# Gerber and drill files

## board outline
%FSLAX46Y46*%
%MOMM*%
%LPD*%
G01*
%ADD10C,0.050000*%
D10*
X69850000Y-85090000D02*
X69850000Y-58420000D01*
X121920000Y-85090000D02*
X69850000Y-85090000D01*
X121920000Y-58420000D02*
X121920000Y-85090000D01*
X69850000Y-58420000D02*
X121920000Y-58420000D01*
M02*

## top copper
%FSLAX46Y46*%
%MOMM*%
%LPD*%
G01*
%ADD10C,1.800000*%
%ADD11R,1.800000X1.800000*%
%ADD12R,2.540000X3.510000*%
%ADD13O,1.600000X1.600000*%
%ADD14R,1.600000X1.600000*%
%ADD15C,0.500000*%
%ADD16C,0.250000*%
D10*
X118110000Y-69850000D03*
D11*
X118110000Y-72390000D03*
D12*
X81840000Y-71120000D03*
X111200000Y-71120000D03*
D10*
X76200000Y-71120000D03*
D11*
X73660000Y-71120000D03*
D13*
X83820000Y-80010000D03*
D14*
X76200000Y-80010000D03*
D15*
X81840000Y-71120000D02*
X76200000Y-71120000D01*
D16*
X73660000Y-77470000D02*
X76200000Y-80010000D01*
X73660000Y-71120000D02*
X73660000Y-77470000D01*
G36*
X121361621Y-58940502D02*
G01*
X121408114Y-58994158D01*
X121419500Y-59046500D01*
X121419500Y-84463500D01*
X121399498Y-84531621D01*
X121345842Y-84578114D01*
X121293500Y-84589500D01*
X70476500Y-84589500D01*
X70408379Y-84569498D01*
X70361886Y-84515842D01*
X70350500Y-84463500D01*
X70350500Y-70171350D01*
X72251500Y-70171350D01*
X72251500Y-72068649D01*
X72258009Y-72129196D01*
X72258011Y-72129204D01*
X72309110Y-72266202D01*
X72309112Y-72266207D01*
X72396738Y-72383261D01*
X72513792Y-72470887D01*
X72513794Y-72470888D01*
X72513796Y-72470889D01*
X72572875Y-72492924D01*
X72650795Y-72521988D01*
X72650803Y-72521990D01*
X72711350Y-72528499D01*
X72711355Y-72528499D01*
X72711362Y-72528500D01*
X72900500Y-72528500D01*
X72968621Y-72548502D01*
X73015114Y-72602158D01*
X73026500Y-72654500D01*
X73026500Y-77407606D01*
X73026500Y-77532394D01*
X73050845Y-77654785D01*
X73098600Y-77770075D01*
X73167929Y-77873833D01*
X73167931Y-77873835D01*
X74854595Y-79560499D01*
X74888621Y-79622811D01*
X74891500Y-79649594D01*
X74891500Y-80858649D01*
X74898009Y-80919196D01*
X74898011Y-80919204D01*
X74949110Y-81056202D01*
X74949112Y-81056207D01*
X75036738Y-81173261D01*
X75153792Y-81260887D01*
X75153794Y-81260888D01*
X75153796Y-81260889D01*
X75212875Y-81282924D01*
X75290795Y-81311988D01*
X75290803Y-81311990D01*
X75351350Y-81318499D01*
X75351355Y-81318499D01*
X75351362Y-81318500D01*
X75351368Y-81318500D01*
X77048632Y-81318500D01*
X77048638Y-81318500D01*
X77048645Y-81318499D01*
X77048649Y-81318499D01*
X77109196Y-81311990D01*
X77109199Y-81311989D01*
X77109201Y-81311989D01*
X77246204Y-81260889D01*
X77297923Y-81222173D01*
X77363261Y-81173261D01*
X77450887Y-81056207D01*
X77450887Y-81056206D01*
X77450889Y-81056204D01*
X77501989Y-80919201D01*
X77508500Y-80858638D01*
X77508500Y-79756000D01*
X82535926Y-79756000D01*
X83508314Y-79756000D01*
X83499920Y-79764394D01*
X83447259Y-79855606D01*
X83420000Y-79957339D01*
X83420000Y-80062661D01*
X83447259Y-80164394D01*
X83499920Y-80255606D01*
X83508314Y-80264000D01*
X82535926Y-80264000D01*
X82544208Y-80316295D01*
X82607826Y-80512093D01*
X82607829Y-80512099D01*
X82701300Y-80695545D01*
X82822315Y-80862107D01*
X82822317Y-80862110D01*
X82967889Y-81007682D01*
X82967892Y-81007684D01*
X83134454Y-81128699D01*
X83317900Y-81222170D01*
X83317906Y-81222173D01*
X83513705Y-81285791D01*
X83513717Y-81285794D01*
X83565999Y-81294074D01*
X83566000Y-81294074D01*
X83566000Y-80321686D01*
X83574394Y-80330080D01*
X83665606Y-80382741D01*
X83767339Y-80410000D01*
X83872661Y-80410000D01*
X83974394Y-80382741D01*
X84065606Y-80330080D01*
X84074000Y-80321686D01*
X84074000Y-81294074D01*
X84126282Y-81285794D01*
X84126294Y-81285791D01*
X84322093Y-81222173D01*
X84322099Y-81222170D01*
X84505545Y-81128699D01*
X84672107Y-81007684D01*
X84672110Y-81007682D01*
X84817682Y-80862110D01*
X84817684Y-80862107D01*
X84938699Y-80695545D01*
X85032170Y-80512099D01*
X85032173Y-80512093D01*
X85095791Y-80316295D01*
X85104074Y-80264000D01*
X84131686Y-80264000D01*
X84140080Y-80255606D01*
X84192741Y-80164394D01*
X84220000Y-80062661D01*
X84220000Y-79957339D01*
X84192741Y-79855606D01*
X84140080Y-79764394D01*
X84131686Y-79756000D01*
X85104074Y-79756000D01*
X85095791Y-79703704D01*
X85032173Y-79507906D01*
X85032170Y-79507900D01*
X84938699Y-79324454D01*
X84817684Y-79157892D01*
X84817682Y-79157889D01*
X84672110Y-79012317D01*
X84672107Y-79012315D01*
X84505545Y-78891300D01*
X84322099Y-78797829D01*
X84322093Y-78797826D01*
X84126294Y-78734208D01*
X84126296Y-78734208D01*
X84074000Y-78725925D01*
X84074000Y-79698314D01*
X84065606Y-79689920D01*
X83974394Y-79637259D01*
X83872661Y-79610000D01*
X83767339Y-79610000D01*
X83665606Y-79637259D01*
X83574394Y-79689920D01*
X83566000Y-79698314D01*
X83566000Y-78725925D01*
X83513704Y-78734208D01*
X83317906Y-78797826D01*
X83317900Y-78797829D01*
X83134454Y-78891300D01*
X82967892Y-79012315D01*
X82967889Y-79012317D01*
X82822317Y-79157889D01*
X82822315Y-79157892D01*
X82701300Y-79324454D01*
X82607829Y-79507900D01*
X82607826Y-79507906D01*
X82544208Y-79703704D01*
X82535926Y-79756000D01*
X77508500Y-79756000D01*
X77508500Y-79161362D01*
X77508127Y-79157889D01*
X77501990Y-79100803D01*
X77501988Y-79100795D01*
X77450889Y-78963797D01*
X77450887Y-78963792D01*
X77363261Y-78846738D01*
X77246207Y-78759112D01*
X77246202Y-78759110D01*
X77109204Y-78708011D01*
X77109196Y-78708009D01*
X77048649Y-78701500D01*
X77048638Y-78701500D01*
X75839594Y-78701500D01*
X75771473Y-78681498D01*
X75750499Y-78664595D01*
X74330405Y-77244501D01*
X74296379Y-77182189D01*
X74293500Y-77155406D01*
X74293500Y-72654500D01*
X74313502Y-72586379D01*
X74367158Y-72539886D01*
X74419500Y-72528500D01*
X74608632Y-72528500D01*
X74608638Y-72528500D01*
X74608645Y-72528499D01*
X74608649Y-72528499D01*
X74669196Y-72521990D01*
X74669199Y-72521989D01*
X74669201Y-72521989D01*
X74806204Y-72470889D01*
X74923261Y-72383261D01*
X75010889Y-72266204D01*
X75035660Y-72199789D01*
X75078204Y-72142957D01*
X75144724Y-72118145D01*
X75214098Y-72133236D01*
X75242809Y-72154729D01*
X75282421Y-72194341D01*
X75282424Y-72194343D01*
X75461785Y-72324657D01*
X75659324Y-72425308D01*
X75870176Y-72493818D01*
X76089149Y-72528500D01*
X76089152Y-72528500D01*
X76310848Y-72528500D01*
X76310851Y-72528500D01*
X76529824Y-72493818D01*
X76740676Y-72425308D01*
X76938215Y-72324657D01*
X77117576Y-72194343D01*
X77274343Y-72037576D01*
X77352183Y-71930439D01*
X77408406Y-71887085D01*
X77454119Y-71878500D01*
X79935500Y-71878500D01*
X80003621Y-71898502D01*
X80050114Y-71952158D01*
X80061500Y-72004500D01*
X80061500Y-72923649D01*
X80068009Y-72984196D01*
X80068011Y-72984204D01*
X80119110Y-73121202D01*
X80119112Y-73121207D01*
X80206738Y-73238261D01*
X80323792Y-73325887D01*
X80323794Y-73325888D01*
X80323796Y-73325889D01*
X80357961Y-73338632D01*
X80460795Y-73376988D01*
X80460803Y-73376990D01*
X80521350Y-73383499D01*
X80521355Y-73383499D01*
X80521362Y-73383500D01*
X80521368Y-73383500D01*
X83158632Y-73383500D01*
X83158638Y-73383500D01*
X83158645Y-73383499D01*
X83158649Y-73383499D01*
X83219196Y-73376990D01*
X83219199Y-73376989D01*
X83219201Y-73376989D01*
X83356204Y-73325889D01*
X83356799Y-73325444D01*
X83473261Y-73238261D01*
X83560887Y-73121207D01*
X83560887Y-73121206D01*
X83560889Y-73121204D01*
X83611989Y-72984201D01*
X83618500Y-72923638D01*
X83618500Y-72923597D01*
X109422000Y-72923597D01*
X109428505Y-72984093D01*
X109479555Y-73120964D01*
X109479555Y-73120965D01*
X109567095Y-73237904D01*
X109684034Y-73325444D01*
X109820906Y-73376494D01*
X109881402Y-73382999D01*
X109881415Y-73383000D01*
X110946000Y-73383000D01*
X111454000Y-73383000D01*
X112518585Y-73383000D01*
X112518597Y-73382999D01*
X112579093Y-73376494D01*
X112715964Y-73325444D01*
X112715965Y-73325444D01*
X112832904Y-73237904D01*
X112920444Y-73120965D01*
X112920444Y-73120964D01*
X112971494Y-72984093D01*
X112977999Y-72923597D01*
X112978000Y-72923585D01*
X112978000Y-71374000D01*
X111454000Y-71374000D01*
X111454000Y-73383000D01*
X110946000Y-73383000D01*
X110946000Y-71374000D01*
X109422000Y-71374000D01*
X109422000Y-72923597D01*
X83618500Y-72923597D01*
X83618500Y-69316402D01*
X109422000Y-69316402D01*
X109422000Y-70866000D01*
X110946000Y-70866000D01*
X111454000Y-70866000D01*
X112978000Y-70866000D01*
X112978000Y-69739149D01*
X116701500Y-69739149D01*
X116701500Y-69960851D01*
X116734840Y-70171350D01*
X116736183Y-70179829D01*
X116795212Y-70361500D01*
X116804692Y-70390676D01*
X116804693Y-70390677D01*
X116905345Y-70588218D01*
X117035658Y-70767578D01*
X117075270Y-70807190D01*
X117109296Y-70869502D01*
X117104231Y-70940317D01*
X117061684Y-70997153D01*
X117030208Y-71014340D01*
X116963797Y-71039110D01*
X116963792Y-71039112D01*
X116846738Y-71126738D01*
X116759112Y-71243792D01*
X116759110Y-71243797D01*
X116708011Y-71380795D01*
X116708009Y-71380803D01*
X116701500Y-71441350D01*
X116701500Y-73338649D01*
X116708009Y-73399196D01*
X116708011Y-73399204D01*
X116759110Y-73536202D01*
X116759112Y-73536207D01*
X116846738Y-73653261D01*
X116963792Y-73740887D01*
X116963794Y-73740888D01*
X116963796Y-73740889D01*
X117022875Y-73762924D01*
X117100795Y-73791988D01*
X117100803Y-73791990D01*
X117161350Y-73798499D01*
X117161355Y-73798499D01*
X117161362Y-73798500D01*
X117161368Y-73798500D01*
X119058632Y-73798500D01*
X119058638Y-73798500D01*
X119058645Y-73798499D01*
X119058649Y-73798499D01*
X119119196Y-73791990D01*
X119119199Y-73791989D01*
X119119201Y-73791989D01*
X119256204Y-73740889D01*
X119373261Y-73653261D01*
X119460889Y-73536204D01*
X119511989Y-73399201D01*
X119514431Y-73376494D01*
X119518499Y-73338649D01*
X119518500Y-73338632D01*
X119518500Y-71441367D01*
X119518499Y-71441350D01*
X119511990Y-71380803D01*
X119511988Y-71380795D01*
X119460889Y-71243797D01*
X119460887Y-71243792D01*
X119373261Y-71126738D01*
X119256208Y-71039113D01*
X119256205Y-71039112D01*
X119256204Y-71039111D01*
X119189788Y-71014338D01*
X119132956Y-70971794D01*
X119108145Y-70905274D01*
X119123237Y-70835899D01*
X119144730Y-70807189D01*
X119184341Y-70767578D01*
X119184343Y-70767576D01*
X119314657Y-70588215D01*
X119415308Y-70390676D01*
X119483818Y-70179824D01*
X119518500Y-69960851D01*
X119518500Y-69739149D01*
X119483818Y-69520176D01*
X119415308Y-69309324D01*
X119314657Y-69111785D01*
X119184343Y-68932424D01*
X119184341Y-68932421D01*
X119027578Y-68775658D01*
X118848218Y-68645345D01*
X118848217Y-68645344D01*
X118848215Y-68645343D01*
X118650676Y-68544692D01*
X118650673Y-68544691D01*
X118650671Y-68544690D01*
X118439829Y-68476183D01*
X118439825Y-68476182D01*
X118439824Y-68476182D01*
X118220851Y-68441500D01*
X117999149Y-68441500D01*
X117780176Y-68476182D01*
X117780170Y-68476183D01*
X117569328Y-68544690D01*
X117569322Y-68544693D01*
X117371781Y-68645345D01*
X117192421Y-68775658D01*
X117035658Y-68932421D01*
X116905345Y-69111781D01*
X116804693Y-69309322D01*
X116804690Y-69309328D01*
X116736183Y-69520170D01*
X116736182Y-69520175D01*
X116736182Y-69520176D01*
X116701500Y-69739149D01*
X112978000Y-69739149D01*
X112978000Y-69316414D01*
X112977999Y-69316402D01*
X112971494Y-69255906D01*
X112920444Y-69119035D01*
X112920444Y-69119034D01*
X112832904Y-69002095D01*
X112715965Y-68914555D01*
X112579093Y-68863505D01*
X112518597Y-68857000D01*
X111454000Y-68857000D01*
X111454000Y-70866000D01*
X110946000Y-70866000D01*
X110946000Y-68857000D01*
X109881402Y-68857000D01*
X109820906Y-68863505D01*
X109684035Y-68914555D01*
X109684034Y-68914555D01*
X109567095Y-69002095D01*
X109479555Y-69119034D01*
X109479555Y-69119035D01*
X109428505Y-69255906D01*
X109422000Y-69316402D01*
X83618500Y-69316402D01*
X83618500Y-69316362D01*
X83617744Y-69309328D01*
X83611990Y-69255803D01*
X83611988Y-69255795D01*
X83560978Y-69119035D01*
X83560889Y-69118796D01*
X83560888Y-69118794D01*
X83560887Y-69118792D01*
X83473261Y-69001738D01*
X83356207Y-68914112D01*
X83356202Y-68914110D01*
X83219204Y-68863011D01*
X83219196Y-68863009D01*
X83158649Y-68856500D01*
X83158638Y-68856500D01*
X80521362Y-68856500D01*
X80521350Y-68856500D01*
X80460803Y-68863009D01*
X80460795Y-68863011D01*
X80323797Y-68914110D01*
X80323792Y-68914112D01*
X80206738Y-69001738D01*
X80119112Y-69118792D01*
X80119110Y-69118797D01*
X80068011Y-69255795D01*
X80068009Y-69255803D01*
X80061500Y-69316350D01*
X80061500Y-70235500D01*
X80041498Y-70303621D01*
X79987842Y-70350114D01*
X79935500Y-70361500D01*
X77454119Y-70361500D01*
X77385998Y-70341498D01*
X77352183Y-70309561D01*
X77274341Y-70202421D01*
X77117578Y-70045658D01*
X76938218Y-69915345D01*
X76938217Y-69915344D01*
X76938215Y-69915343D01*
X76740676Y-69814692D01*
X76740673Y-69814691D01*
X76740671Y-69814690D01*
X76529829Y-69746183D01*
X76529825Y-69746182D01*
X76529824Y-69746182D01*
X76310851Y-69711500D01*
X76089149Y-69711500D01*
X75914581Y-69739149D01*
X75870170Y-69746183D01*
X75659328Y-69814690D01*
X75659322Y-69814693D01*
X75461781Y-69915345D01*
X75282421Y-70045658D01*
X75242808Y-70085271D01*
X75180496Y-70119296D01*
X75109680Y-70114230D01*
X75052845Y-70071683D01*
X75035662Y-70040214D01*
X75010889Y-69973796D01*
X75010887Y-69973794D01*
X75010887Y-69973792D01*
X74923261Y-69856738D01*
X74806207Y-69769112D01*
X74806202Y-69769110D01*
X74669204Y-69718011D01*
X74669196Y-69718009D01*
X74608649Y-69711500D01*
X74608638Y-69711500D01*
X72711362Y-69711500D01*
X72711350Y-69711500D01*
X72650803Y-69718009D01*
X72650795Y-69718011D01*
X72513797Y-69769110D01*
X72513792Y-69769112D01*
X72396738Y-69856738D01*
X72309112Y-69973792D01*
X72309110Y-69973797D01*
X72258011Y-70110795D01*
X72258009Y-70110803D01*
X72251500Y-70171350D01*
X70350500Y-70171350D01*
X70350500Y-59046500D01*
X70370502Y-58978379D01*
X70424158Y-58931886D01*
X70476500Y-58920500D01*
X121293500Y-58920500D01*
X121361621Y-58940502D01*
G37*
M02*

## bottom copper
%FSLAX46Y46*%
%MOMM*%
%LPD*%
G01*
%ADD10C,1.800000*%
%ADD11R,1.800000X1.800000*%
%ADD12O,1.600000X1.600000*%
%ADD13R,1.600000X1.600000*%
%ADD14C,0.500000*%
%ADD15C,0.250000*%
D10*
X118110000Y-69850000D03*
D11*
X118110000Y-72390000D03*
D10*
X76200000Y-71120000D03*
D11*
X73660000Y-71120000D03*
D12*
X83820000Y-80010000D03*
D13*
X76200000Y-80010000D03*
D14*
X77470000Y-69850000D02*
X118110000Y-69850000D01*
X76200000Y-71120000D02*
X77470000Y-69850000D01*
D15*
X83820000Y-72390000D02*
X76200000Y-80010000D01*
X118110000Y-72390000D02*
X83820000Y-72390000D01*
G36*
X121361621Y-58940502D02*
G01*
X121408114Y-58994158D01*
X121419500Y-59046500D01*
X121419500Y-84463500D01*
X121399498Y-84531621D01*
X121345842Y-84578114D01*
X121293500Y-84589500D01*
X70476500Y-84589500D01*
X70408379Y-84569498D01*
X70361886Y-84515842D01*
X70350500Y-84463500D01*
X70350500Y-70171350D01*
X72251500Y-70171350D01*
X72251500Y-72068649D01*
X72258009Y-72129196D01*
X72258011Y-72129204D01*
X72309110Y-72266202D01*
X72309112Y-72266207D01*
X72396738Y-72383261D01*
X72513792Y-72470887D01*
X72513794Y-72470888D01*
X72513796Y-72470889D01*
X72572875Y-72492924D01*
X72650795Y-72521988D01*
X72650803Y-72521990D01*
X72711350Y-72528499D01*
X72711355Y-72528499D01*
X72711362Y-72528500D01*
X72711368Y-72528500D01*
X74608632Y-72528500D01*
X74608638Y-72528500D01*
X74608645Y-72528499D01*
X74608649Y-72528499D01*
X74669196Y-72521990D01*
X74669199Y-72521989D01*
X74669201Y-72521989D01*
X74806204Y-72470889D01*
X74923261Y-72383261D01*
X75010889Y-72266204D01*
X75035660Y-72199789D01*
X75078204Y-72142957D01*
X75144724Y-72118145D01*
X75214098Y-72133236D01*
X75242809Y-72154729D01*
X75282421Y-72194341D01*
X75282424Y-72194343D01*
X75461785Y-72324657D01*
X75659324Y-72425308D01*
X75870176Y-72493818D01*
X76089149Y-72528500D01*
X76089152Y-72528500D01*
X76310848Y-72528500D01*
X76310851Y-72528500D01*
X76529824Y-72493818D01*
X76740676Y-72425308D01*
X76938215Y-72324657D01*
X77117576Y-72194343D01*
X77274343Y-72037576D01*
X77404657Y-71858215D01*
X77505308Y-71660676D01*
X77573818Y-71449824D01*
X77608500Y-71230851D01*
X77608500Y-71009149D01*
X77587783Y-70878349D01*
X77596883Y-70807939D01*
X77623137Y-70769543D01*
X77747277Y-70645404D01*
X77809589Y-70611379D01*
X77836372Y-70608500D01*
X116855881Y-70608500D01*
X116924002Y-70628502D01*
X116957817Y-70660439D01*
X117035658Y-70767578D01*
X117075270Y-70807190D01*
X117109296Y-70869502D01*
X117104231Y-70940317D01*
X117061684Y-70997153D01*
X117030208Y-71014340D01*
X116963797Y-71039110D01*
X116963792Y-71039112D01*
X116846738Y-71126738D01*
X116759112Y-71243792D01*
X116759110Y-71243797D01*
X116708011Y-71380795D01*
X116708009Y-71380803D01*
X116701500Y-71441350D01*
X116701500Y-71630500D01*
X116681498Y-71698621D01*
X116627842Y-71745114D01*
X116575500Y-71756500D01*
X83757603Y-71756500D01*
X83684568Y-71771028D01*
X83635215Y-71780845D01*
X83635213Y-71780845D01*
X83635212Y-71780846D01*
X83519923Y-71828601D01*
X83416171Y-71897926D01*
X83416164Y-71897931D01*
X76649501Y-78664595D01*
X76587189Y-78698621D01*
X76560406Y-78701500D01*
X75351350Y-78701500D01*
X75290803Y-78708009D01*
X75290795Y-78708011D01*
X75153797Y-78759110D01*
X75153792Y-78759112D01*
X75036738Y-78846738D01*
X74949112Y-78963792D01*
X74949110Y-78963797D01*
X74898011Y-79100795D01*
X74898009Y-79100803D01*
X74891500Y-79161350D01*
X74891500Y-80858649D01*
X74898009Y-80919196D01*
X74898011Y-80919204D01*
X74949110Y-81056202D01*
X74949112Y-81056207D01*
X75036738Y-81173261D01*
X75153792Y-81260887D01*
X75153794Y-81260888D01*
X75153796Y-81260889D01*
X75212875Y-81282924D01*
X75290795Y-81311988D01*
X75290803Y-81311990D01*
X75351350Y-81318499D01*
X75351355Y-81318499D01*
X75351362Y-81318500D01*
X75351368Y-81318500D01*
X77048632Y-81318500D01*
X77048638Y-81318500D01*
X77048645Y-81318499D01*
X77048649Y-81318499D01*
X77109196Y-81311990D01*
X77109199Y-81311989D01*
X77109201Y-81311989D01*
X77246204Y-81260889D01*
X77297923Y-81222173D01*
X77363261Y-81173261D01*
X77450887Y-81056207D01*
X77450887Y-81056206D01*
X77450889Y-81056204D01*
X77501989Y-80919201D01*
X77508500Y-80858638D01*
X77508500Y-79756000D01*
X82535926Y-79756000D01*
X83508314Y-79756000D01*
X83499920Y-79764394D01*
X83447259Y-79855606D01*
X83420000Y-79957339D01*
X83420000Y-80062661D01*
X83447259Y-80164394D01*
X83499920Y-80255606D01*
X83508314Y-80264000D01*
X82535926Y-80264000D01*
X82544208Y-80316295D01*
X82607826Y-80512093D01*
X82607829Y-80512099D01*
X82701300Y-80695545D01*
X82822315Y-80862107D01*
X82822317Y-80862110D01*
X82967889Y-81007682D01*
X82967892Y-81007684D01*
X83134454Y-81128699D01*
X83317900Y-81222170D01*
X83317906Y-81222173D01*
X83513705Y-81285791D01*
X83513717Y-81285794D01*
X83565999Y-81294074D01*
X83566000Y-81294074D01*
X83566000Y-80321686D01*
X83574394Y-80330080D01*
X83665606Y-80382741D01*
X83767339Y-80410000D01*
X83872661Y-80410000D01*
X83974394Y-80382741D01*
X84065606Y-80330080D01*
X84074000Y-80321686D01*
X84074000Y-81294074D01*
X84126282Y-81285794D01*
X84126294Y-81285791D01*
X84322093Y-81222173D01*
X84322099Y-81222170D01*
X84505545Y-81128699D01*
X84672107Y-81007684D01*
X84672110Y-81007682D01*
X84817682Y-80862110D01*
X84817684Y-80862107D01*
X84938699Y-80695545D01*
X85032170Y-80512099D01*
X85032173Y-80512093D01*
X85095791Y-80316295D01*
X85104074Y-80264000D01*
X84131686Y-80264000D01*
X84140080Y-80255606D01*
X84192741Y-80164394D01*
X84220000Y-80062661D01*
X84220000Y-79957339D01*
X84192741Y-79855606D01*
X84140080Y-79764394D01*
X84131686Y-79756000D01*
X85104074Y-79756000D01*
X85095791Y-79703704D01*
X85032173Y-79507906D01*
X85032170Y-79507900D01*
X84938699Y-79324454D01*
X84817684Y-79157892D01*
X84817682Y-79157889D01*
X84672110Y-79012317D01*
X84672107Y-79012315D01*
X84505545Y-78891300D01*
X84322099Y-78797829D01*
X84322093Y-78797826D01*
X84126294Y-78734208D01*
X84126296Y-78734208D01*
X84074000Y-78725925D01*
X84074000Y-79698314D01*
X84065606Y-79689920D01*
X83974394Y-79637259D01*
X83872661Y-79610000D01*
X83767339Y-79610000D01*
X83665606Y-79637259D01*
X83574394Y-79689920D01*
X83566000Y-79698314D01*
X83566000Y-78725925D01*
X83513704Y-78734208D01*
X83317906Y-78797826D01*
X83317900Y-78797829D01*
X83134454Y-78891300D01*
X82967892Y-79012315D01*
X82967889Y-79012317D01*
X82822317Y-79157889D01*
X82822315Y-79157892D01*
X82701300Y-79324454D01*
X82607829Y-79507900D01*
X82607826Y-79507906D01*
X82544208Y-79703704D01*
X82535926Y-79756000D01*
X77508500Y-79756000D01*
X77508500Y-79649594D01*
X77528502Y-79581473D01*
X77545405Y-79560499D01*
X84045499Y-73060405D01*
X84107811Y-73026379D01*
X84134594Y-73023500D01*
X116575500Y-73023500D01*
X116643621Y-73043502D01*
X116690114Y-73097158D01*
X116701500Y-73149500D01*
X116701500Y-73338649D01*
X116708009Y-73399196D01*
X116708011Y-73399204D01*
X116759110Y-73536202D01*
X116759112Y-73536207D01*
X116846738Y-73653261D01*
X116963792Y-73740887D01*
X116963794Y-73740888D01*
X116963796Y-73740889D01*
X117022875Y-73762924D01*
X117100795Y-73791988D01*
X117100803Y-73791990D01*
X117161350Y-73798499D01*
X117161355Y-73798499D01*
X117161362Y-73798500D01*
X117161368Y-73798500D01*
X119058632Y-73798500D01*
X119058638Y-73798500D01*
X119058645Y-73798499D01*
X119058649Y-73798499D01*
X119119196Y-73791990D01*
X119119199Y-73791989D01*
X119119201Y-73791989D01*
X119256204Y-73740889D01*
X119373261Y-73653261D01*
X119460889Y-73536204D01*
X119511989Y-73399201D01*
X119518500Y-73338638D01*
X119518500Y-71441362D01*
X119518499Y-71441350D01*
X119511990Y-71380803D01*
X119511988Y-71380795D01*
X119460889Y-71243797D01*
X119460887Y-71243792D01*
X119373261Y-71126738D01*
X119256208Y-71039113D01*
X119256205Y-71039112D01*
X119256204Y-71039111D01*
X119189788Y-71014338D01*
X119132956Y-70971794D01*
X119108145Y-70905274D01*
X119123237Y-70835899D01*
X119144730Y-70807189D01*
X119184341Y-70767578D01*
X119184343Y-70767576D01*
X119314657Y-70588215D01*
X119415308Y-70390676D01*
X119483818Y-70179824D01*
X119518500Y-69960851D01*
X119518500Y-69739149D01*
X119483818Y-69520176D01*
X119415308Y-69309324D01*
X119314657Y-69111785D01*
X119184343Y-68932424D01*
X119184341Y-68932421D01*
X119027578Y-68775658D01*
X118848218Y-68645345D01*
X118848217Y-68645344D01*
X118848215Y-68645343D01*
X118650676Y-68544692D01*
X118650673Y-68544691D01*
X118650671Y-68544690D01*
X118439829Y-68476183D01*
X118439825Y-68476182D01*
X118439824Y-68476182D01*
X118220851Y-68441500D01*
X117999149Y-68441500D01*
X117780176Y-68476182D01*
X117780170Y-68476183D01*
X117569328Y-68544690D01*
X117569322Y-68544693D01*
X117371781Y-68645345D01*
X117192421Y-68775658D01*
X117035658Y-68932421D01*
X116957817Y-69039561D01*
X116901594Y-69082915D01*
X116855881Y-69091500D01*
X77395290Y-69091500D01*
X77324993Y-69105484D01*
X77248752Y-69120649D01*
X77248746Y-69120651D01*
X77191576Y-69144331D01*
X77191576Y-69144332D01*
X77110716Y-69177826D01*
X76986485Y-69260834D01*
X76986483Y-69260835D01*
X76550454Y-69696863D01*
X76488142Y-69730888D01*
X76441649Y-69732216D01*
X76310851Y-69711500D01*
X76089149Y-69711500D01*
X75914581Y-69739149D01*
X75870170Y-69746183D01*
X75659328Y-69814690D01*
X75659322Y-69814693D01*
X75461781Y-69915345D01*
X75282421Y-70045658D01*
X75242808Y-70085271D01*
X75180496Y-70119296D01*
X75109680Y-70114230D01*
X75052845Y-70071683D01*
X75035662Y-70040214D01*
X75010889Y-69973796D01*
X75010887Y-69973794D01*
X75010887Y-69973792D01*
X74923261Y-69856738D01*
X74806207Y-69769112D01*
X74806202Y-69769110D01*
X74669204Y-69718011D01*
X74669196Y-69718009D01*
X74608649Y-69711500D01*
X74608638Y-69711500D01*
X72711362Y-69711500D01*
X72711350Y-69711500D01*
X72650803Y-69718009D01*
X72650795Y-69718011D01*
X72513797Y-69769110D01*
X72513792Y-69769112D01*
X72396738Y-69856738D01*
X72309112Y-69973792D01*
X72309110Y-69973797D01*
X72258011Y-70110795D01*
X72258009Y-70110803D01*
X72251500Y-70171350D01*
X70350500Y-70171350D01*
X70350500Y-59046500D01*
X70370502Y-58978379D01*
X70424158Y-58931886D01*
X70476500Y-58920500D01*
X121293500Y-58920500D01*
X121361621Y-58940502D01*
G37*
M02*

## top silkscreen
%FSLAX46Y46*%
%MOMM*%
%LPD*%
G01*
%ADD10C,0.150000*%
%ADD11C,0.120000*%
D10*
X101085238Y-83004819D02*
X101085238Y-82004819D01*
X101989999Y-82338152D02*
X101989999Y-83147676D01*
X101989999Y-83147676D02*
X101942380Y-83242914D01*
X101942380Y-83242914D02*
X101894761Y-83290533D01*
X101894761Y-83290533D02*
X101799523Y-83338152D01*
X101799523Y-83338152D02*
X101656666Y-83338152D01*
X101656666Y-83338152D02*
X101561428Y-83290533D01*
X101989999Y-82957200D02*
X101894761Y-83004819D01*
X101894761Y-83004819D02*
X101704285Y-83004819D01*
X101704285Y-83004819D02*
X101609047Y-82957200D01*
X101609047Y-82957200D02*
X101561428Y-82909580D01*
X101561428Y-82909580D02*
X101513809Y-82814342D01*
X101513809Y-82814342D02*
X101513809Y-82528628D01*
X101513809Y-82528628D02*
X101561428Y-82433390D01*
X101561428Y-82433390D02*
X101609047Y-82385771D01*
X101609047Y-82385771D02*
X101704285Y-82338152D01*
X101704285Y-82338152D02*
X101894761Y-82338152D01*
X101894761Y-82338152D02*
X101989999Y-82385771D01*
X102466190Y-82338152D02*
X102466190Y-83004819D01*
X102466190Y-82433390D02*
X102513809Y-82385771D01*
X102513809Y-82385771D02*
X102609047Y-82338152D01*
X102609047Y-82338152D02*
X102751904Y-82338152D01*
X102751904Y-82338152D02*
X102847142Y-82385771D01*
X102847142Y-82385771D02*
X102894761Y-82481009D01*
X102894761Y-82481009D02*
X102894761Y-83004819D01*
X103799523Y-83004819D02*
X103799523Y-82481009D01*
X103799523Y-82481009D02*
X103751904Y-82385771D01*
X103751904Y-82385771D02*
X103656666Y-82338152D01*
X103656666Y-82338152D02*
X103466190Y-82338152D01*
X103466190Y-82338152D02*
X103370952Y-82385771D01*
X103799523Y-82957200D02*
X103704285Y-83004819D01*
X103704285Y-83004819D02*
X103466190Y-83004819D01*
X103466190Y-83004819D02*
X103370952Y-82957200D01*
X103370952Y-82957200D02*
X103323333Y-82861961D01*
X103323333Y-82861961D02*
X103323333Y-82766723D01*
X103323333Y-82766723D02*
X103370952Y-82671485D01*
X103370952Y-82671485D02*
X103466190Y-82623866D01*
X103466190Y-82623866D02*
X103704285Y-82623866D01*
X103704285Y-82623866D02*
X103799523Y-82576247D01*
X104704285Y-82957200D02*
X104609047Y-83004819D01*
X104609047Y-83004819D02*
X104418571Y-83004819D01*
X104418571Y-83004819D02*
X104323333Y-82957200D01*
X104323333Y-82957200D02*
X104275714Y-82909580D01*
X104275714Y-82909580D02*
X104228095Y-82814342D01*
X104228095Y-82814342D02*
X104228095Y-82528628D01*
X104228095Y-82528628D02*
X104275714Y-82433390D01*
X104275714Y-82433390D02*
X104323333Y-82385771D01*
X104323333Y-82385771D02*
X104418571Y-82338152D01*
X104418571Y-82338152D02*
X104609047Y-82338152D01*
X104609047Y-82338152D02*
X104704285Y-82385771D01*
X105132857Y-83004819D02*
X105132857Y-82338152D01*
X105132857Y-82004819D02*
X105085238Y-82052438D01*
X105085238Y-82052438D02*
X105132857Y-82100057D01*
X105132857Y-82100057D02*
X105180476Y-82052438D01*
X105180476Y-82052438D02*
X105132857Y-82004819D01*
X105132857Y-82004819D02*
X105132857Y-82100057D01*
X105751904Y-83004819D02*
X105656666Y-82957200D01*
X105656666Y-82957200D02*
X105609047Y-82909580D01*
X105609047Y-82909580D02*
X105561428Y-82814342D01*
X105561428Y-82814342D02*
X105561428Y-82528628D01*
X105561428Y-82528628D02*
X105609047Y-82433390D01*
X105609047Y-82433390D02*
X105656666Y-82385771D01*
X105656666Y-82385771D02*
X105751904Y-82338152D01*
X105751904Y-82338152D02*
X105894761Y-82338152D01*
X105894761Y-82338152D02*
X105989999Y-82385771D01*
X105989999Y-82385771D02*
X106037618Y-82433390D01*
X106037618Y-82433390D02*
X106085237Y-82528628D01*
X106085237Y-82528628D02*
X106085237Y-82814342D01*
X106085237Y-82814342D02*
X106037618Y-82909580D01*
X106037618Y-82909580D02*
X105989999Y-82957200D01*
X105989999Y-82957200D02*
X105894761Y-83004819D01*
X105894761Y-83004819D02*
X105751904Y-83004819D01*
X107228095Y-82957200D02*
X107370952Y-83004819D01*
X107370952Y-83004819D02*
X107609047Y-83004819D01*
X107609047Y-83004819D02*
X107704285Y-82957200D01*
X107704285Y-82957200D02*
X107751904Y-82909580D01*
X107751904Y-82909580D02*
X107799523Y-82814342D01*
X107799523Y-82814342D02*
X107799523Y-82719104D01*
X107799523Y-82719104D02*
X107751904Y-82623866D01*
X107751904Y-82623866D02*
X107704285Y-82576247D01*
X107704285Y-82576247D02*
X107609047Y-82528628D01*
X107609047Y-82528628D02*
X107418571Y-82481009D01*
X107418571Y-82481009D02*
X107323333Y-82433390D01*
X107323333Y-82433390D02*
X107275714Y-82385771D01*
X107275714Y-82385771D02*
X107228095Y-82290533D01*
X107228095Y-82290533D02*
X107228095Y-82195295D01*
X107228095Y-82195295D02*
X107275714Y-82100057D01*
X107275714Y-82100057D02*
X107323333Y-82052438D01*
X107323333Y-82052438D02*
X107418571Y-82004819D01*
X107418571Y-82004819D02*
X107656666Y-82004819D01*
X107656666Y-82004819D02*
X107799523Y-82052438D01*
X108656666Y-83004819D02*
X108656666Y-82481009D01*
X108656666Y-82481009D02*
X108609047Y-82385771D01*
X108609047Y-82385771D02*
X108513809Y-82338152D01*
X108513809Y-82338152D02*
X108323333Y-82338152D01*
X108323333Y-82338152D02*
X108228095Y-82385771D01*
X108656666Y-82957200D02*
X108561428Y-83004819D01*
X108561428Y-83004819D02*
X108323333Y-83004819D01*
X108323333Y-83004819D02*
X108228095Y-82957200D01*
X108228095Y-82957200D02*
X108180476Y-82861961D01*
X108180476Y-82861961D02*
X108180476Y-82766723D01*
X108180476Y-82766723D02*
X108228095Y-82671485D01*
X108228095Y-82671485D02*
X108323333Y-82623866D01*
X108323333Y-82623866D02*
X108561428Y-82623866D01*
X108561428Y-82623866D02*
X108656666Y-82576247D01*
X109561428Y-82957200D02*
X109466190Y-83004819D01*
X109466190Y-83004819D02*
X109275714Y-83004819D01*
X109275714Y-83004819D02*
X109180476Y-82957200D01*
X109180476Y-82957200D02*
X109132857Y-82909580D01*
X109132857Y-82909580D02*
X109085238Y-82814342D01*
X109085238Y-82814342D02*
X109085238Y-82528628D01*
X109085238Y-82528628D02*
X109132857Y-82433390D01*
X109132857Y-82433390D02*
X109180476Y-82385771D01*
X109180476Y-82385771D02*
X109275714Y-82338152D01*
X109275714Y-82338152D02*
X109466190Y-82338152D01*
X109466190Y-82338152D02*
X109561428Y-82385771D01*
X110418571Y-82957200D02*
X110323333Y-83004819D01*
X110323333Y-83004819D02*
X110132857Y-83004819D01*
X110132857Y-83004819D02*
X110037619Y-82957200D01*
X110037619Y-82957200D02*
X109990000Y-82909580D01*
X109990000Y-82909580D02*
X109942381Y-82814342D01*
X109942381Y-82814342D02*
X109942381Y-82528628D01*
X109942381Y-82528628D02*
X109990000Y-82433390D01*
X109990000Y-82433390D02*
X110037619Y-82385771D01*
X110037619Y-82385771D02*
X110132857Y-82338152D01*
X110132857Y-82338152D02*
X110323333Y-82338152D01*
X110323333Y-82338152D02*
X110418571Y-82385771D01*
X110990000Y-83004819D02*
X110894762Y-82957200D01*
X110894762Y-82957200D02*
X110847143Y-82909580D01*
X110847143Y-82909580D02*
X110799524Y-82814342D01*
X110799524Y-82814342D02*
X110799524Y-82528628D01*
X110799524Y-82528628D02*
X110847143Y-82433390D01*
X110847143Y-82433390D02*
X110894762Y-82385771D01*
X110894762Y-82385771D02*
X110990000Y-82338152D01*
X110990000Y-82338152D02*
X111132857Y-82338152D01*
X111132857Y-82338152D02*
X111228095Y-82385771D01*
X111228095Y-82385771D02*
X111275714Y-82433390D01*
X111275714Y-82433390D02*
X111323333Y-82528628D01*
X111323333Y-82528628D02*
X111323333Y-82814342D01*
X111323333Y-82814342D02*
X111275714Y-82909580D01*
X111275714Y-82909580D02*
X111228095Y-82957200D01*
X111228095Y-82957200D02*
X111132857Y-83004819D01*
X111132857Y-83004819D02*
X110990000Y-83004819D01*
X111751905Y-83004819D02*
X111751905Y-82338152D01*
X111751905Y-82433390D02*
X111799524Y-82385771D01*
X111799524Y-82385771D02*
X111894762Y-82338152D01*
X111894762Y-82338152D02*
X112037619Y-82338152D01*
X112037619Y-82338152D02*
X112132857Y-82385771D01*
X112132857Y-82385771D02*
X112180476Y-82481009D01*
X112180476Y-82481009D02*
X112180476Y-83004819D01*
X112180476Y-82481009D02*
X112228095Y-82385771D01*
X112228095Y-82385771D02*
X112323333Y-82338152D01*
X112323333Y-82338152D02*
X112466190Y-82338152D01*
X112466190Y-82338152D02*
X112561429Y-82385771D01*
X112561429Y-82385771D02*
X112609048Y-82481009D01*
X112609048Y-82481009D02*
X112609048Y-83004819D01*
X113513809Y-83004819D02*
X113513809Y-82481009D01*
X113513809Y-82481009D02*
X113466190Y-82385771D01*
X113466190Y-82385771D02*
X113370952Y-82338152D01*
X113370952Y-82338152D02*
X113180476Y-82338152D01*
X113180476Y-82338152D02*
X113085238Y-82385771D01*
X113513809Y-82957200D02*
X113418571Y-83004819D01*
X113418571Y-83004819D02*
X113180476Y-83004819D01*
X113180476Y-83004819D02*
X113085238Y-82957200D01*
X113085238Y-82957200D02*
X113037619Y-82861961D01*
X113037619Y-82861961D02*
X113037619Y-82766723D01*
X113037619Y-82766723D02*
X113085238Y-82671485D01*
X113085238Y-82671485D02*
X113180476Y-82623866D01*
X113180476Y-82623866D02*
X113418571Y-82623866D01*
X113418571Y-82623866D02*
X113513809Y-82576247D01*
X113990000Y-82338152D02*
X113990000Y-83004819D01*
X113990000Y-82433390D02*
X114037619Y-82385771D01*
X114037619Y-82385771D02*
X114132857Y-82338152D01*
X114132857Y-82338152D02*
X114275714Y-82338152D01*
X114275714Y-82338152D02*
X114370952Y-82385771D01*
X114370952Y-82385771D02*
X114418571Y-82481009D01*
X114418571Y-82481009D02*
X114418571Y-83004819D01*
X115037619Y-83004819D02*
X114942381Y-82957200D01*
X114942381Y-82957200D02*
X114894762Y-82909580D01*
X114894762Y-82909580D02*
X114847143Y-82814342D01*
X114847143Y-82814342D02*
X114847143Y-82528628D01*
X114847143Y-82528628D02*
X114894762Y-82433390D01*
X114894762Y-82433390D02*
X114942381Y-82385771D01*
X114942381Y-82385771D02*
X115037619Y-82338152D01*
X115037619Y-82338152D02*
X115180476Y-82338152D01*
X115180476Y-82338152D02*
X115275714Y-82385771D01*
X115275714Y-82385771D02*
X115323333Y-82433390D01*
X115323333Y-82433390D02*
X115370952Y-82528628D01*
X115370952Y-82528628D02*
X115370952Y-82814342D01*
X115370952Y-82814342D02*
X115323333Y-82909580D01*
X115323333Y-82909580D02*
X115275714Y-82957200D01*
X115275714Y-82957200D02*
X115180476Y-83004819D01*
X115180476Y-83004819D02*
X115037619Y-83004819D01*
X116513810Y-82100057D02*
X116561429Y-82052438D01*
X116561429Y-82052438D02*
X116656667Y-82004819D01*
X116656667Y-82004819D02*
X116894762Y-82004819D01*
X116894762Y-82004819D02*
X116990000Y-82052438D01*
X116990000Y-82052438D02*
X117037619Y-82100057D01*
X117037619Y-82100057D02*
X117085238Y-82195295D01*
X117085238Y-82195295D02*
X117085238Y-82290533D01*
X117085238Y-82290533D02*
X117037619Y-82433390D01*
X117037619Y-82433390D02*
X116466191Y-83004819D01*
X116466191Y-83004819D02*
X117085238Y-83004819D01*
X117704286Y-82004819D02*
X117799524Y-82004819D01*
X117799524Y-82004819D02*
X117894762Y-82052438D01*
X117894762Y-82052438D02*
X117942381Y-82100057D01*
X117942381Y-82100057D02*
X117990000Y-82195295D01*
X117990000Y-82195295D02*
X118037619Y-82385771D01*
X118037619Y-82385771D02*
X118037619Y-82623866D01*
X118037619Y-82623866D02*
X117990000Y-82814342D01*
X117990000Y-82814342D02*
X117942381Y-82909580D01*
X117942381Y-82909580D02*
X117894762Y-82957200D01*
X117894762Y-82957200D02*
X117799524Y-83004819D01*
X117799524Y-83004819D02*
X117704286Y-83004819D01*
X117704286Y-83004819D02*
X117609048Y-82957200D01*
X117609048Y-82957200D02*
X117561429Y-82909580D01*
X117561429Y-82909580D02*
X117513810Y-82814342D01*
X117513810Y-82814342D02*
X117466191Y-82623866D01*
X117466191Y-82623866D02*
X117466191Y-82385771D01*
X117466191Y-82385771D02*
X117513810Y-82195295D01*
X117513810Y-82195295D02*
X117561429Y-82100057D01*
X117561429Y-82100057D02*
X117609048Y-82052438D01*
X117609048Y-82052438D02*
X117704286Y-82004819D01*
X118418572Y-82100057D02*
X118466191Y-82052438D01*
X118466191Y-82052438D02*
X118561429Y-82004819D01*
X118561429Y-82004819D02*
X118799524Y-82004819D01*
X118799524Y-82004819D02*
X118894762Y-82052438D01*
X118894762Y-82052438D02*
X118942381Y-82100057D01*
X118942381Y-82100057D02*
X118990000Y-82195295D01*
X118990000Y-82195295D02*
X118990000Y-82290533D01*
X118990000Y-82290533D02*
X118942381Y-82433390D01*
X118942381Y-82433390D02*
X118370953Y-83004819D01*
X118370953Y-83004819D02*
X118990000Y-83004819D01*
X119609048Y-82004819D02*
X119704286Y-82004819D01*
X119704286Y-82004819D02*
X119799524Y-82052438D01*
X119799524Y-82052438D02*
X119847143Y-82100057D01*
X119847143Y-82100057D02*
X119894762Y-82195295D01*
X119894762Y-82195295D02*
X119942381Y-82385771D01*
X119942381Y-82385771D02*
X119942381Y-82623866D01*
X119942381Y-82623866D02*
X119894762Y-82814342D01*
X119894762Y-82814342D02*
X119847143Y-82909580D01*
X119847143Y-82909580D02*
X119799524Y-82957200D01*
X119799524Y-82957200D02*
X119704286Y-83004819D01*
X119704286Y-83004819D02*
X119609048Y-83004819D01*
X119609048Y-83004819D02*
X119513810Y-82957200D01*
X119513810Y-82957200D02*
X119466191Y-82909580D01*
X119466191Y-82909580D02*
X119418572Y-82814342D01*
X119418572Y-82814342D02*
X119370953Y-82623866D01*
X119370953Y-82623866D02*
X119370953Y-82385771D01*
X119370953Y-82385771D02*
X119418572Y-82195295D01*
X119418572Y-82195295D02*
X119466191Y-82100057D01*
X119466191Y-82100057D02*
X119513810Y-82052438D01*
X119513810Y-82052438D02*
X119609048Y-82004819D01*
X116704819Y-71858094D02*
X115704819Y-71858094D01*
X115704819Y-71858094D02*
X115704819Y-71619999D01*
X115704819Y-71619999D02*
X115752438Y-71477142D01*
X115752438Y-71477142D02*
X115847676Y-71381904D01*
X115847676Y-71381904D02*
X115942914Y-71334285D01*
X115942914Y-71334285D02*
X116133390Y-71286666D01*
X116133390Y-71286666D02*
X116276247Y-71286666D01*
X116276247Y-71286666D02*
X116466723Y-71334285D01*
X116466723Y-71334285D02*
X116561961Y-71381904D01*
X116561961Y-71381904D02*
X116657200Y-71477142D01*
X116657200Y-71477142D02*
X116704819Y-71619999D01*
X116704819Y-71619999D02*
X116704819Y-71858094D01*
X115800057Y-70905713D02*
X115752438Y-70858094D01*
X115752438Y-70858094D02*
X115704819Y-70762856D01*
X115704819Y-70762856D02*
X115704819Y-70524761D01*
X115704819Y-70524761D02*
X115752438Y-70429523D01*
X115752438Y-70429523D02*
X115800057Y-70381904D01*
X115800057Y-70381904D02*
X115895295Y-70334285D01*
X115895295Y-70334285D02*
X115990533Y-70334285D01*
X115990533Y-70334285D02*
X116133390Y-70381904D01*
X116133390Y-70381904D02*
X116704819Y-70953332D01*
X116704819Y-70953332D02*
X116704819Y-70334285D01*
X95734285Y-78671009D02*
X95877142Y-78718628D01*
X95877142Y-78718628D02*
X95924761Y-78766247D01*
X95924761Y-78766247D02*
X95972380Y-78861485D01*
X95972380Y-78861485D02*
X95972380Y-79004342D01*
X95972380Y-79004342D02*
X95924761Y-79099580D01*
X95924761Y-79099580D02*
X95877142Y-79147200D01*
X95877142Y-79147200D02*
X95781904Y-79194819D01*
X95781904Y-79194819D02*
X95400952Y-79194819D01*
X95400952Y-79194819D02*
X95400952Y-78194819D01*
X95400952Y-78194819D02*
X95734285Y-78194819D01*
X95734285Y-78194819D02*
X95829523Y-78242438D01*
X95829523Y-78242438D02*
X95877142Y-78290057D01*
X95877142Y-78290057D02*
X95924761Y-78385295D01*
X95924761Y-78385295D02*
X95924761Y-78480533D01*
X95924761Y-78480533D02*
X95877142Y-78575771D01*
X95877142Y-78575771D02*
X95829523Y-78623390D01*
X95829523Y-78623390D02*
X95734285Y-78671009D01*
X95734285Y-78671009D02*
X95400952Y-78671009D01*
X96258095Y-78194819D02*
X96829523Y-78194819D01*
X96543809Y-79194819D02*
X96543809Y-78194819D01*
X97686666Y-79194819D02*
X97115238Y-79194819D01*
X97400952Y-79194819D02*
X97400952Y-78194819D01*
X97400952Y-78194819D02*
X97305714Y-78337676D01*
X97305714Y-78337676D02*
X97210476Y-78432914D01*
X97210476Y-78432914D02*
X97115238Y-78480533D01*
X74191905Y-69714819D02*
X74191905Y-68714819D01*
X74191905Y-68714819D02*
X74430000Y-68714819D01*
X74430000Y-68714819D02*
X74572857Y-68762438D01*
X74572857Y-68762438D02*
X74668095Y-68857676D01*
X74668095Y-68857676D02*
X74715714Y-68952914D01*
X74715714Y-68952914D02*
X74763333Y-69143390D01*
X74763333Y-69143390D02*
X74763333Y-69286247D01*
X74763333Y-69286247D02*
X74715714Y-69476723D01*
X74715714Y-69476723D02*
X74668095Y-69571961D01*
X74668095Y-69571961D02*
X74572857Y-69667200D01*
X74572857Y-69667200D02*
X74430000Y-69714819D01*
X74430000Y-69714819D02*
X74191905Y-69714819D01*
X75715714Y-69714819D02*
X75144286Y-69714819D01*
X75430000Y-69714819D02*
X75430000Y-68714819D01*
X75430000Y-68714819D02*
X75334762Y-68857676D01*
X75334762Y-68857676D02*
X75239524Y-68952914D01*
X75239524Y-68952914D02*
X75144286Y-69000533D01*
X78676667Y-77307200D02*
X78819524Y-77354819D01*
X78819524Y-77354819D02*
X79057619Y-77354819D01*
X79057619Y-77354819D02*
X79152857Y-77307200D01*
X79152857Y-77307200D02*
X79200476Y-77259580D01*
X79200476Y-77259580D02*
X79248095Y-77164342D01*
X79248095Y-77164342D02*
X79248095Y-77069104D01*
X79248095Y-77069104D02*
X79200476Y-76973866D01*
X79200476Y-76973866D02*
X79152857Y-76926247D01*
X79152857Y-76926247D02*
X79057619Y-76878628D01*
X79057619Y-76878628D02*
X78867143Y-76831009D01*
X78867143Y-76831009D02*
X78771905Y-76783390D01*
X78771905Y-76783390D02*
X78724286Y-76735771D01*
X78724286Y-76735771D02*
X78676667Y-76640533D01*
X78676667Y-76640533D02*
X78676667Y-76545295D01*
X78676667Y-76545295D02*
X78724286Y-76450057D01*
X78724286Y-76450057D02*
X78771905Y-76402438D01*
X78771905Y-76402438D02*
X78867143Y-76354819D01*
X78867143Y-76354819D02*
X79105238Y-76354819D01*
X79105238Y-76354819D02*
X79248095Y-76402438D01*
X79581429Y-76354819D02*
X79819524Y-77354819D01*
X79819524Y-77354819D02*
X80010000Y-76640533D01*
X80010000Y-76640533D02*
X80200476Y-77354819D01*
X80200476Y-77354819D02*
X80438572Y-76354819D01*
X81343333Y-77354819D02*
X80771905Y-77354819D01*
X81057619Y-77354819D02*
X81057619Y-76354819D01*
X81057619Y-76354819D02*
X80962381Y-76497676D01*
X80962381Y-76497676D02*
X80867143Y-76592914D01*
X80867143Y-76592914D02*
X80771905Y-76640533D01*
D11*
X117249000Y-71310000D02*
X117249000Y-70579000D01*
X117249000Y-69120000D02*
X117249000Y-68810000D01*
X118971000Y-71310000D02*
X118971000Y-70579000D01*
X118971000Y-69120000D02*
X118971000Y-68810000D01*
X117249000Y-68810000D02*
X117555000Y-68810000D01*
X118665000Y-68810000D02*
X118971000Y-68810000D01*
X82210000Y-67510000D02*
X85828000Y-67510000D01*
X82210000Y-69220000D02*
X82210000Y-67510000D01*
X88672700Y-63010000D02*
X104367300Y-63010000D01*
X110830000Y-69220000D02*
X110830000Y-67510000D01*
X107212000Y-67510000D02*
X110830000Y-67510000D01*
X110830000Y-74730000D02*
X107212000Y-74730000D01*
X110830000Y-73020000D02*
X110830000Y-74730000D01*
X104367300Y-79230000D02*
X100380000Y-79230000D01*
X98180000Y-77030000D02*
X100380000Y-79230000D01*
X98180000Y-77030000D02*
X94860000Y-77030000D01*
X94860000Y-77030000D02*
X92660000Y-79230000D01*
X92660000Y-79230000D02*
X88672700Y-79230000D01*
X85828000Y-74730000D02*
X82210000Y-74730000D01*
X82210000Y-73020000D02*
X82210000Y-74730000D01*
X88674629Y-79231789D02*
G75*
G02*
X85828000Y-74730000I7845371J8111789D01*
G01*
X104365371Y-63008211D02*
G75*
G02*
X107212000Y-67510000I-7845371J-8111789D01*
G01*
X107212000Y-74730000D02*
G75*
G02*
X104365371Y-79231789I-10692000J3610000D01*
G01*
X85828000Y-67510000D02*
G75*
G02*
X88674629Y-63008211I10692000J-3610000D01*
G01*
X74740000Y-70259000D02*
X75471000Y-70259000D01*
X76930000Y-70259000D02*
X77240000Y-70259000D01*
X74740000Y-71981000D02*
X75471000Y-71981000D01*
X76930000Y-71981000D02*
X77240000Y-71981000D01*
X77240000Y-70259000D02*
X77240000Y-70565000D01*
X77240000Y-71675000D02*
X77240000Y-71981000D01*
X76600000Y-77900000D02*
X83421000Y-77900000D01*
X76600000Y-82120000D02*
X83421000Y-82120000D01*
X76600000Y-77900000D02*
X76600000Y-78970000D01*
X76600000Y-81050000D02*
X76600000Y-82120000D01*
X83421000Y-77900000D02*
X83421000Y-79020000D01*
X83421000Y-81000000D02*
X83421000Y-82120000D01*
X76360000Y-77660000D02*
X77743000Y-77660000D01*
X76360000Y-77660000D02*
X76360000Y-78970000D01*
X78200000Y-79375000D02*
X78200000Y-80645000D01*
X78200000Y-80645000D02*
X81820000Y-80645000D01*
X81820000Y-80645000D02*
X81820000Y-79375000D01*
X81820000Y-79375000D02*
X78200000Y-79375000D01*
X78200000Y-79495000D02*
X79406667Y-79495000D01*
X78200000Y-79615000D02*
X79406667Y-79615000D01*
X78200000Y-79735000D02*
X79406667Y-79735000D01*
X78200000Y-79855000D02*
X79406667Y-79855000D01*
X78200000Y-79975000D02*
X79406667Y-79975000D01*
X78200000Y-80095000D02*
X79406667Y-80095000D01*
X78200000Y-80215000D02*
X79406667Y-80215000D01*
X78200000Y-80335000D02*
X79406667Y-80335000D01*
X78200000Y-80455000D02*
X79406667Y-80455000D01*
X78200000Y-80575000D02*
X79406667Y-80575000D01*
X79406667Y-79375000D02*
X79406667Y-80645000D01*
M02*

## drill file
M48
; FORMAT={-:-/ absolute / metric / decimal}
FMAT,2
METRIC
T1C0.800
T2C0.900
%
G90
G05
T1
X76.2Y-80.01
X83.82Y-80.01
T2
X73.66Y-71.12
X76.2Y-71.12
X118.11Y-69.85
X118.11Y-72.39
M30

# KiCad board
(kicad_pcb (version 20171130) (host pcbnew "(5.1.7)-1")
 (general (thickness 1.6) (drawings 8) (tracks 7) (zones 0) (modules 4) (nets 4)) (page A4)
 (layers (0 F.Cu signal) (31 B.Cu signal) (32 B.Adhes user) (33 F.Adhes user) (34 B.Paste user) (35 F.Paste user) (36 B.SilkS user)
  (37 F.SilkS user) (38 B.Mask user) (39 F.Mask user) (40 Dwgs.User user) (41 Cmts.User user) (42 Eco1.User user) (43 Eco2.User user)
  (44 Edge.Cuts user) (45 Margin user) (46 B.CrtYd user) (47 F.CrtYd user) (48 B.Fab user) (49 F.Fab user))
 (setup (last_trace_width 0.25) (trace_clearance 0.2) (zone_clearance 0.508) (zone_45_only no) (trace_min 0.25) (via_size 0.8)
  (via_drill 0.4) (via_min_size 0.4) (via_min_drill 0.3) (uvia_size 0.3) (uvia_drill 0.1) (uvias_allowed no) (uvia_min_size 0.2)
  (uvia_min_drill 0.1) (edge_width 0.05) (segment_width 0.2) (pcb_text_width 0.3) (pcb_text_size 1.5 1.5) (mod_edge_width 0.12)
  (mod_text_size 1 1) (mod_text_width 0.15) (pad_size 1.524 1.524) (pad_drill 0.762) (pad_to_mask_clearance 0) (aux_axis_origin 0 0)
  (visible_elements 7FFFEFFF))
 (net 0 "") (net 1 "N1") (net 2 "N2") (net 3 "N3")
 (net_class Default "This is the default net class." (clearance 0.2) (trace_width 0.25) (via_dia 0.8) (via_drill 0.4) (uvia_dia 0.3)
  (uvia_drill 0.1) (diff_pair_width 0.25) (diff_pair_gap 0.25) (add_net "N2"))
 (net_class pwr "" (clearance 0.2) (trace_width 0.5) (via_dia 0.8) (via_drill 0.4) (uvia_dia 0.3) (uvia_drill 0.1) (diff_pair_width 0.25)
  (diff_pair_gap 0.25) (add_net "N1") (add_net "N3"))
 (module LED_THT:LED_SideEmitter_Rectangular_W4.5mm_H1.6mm (layer F.Cu) (at 118.11 72.39 90)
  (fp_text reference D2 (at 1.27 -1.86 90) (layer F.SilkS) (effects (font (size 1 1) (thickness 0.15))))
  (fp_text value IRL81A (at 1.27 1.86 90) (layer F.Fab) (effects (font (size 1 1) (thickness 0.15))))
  (fp_line (start 1.08 -0.861) (end 1.811 -0.861) (layer F.SilkS) (width 0.12))
  (fp_line (start 3.27 -0.861) (end 3.58 -0.861) (layer F.SilkS) (width 0.12))
  (fp_line (start 1.08 0.861) (end 1.811 0.861) (layer F.SilkS) (width 0.12))
  (fp_line (start 3.27 0.861) (end 3.58 0.861) (layer F.SilkS) (width 0.12))
  (fp_line (start 3.58 -0.861) (end 3.58 -0.555) (layer F.SilkS) (width 0.12))
  (fp_line (start 3.58 0.555) (end 3.58 0.861) (layer F.SilkS) (width 0.12))
  (pad 2 thru_hole circle (at 2.54 0 90) (size 1.8 1.8) (drill 0.9) (layers *.Cu *.Mask) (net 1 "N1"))
  (pad 1 thru_hole rect (at 0 0 90) (size 1.8 1.8) (drill 0.9) (layers *.Cu *.Mask) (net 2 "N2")))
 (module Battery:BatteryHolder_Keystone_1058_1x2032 (layer F.Cu) (at 96.52 71.12)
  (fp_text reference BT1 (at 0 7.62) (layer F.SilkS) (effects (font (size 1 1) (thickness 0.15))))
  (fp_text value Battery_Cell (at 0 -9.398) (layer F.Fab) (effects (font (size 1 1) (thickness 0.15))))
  (fp_line (start -14.31 -3.61) (end -10.692 -3.61) (layer F.SilkS) (width 0.12))
  (fp_line (start -14.31 -1.9) (end -14.31 -3.61) (layer F.SilkS) (width 0.12))
  (fp_line (start -7.8473 -8.11) (end 7.8473 -8.11) (layer F.SilkS) (width 0.12))
  (fp_line (start 14.31 -1.9) (end 14.31 -3.61) (layer F.SilkS) (width 0.12))
  (fp_line (start 10.692 -3.61) (end 14.31 -3.61) (layer F.SilkS) (width 0.12))
  (fp_line (start 14.31 3.61) (end 10.692 3.61) (layer F.SilkS) (width 0.12))
  (fp_line (start 14.31 1.9) (end 14.31 3.61) (layer F.SilkS) (width 0.12))
  (fp_line (start 7.8473 8.11) (end 3.86 8.11) (layer F.SilkS) (width 0.12))
  (fp_line (start 1.66 5.91) (end 3.86 8.11) (layer F.SilkS) (width 0.12))
  (fp_line (start 1.66 5.91) (end -1.66 5.91) (layer F.SilkS) (width 0.12))
  (fp_line (start -1.66 5.91) (end -3.86 8.11) (layer F.SilkS) (width 0.12))
  (fp_line (start -3.86 8.11) (end -7.8473 8.11) (layer F.SilkS) (width 0.12))
  (fp_line (start -10.692 3.61) (end -14.31 3.61) (layer F.SilkS) (width 0.12))
  (fp_line (start -14.31 1.9) (end -14.31 3.61) (layer F.SilkS) (width 0.12))
  (fp_arc (start 0 0) (end -10.692 3.61) (angle -27.3) (layer F.SilkS) (width 0.12))
  (fp_arc (start 0 0) (end 10.692 -3.61) (angle -27.3) (layer F.SilkS) (width 0.12))
  (fp_arc (start 0 0) (end 10.692 3.61) (angle 27.3) (layer F.SilkS) (width 0.12))
  (fp_arc (start 0 0) (end -10.692 -3.61) (angle 27.3) (layer F.SilkS) (width 0.12))
  (pad 1 smd rect (at -14.68 0) (size 2.54 3.51) (layers F.Cu F.Paste F.Mask) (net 1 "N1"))
  (pad 2 smd rect (at 14.68 0) (size 2.54 3.51) (layers F.Cu F.Paste F.Mask) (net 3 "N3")))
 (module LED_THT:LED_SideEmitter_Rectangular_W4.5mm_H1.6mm (layer F.Cu) (at 73.66 71.12)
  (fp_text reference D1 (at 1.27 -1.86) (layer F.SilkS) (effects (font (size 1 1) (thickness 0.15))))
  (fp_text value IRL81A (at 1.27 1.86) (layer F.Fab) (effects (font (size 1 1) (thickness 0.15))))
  (fp_line (start 1.08 -0.861) (end 1.811 -0.861) (layer F.SilkS) (width 0.12))
  (fp_line (start 3.27 -0.861) (end 3.58 -0.861) (layer F.SilkS) (width 0.12))
  (fp_line (start 1.08 0.861) (end 1.811 0.861) (layer F.SilkS) (width 0.12))
  (fp_line (start 3.27 0.861) (end 3.58 0.861) (layer F.SilkS) (width 0.12))
  (fp_line (start 3.58 -0.861) (end 3.58 -0.555) (layer F.SilkS) (width 0.12))
  (fp_line (start 3.58 0.555) (end 3.58 0.861) (layer F.SilkS) (width 0.12))
  (pad 2 thru_hole circle (at 2.54 0) (size 1.8 1.8) (drill 0.9) (layers *.Cu *.Mask) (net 1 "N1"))
  (pad 1 thru_hole rect (at 0 0) (size 1.8 1.8) (drill 0.9) (layers *.Cu *.Mask) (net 2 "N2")))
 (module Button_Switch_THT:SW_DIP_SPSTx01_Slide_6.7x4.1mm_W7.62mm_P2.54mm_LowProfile (layer F.Cu) (at 76.2 80.01)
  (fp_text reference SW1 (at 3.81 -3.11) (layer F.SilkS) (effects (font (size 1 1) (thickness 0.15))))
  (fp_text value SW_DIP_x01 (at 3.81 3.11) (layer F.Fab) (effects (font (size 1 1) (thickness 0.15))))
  (fp_line (start 0.4 -2.11) (end 7.221 -2.11) (layer F.SilkS) (width 0.12))
  (fp_line (start 0.4 2.11) (end 7.221 2.11) (layer F.SilkS) (width 0.12))
  (fp_line (start 0.4 -2.11) (end 0.4 -1.04) (layer F.SilkS) (width 0.12))
  (fp_line (start 0.4 1.04) (end 0.4 2.11) (layer F.SilkS) (width 0.12))
  (fp_line (start 7.221 -2.11) (end 7.221 -0.99) (layer F.SilkS) (width 0.12))
  (fp_line (start 7.221 0.99) (end 7.221 2.11) (layer F.SilkS) (width 0.12))
  (fp_line (start 0.16 -2.35) (end 1.543 -2.35) (layer F.SilkS) (width 0.12))
  (fp_line (start 0.16 -2.35) (end 0.16 -1.04) (layer F.SilkS) (width 0.12))
  (fp_line (start 2 -0.635) (end 2 0.635) (layer F.SilkS) (width 0.12))
  (fp_line (start 2 0.635) (end 5.62 0.635) (layer F.SilkS) (width 0.12))
  (fp_line (start 5.62 0.635) (end 5.62 -0.635) (layer F.SilkS) (width 0.12))
  (fp_line (start 5.62 -0.635) (end 2 -0.635) (layer F.SilkS) (width 0.12))
  (fp_line (start 2 -0.515) (end 3.206667 -0.515) (layer F.SilkS) (width 0.12))
  (fp_line (start 2 -0.395) (end 3.206667 -0.395) (layer F.SilkS) (width 0.12))
  (fp_line (start 2 -0.275) (end 3.206667 -0.275) (layer F.SilkS) (width 0.12))
  (fp_line (start 2 -0.155) (end 3.206667 -0.155) (layer F.SilkS) (width 0.12))
  (fp_line (start 2 -0.035) (end 3.206667 -0.035) (layer F.SilkS) (width 0.12))
  (fp_line (start 2 0.085) (end 3.206667 0.085) (layer F.SilkS) (width 0.12))
  (fp_line (start 2 0.205) (end 3.206667 0.205) (layer F.SilkS) (width 0.12))
  (fp_line (start 2 0.325) (end 3.206667 0.325) (layer F.SilkS) (width 0.12))
  (fp_line (start 2 0.445) (end 3.206667 0.445) (layer F.SilkS) (width 0.12))
  (fp_line (start 2 0.565) (end 3.206667 0.565) (layer F.SilkS) (width 0.12))
  (fp_line (start 3.206667 -0.635) (end 3.206667 0.635) (layer F.SilkS) (width 0.12))
  (pad 2 thru_hole oval (at 7.62 0) (size 1.6 1.6) (drill 0.8) (layers *.Cu *.Mask) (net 3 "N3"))
  (pad 1 thru_hole rect (at 0 0) (size 1.6 1.6) (drill 0.8) (layers *.Cu *.Mask) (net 2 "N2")))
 (gr_line (start 69.85 85.09) (end 69.85 58.42) (layer Edge.Cuts) (width 0.05))
 (gr_line (start 121.92 85.09) (end 69.85 85.09) (layer Edge.Cuts) (width 0.05))
 (gr_line (start 121.92 58.42) (end 121.92 85.09) (layer Edge.Cuts) (width 0.05))
 (gr_line (start 69.85 58.42) (end 121.92 58.42) (layer Edge.Cuts) (width 0.05))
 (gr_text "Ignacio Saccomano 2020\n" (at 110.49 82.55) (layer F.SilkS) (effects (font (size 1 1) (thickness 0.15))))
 (segment (start 81.84 71.12) (end 76.2 71.12) (width 0.5) (layer F.Cu) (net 1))
 (segment (start 77.47 69.85) (end 118.11 69.85) (width 0.5) (layer B.Cu) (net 1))
 (segment (start 76.2 71.12) (end 77.47 69.85) (width 0.5) (layer B.Cu) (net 1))
 (segment (start 73.66 77.47) (end 76.2 80.01) (width 0.25) (layer F.Cu) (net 2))
 (segment (start 73.66 71.12) (end 73.66 77.47) (width 0.25) (layer F.Cu) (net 2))
 (segment (start 83.82 72.39) (end 76.2 80.01) (width 0.25) (layer B.Cu) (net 2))
 (segment (start 118.11 72.39) (end 83.82 72.39) (width 0.25) (layer B.Cu) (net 2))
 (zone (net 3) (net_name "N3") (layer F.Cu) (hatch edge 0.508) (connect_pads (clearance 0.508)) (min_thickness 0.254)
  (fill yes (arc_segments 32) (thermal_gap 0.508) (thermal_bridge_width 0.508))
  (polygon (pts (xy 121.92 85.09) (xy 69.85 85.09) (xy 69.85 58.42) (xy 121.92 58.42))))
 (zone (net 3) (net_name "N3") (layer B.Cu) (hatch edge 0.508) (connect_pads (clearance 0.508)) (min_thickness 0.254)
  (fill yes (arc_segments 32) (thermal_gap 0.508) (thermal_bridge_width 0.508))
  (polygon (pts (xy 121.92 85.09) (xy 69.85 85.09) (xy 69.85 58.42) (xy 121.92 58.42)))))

